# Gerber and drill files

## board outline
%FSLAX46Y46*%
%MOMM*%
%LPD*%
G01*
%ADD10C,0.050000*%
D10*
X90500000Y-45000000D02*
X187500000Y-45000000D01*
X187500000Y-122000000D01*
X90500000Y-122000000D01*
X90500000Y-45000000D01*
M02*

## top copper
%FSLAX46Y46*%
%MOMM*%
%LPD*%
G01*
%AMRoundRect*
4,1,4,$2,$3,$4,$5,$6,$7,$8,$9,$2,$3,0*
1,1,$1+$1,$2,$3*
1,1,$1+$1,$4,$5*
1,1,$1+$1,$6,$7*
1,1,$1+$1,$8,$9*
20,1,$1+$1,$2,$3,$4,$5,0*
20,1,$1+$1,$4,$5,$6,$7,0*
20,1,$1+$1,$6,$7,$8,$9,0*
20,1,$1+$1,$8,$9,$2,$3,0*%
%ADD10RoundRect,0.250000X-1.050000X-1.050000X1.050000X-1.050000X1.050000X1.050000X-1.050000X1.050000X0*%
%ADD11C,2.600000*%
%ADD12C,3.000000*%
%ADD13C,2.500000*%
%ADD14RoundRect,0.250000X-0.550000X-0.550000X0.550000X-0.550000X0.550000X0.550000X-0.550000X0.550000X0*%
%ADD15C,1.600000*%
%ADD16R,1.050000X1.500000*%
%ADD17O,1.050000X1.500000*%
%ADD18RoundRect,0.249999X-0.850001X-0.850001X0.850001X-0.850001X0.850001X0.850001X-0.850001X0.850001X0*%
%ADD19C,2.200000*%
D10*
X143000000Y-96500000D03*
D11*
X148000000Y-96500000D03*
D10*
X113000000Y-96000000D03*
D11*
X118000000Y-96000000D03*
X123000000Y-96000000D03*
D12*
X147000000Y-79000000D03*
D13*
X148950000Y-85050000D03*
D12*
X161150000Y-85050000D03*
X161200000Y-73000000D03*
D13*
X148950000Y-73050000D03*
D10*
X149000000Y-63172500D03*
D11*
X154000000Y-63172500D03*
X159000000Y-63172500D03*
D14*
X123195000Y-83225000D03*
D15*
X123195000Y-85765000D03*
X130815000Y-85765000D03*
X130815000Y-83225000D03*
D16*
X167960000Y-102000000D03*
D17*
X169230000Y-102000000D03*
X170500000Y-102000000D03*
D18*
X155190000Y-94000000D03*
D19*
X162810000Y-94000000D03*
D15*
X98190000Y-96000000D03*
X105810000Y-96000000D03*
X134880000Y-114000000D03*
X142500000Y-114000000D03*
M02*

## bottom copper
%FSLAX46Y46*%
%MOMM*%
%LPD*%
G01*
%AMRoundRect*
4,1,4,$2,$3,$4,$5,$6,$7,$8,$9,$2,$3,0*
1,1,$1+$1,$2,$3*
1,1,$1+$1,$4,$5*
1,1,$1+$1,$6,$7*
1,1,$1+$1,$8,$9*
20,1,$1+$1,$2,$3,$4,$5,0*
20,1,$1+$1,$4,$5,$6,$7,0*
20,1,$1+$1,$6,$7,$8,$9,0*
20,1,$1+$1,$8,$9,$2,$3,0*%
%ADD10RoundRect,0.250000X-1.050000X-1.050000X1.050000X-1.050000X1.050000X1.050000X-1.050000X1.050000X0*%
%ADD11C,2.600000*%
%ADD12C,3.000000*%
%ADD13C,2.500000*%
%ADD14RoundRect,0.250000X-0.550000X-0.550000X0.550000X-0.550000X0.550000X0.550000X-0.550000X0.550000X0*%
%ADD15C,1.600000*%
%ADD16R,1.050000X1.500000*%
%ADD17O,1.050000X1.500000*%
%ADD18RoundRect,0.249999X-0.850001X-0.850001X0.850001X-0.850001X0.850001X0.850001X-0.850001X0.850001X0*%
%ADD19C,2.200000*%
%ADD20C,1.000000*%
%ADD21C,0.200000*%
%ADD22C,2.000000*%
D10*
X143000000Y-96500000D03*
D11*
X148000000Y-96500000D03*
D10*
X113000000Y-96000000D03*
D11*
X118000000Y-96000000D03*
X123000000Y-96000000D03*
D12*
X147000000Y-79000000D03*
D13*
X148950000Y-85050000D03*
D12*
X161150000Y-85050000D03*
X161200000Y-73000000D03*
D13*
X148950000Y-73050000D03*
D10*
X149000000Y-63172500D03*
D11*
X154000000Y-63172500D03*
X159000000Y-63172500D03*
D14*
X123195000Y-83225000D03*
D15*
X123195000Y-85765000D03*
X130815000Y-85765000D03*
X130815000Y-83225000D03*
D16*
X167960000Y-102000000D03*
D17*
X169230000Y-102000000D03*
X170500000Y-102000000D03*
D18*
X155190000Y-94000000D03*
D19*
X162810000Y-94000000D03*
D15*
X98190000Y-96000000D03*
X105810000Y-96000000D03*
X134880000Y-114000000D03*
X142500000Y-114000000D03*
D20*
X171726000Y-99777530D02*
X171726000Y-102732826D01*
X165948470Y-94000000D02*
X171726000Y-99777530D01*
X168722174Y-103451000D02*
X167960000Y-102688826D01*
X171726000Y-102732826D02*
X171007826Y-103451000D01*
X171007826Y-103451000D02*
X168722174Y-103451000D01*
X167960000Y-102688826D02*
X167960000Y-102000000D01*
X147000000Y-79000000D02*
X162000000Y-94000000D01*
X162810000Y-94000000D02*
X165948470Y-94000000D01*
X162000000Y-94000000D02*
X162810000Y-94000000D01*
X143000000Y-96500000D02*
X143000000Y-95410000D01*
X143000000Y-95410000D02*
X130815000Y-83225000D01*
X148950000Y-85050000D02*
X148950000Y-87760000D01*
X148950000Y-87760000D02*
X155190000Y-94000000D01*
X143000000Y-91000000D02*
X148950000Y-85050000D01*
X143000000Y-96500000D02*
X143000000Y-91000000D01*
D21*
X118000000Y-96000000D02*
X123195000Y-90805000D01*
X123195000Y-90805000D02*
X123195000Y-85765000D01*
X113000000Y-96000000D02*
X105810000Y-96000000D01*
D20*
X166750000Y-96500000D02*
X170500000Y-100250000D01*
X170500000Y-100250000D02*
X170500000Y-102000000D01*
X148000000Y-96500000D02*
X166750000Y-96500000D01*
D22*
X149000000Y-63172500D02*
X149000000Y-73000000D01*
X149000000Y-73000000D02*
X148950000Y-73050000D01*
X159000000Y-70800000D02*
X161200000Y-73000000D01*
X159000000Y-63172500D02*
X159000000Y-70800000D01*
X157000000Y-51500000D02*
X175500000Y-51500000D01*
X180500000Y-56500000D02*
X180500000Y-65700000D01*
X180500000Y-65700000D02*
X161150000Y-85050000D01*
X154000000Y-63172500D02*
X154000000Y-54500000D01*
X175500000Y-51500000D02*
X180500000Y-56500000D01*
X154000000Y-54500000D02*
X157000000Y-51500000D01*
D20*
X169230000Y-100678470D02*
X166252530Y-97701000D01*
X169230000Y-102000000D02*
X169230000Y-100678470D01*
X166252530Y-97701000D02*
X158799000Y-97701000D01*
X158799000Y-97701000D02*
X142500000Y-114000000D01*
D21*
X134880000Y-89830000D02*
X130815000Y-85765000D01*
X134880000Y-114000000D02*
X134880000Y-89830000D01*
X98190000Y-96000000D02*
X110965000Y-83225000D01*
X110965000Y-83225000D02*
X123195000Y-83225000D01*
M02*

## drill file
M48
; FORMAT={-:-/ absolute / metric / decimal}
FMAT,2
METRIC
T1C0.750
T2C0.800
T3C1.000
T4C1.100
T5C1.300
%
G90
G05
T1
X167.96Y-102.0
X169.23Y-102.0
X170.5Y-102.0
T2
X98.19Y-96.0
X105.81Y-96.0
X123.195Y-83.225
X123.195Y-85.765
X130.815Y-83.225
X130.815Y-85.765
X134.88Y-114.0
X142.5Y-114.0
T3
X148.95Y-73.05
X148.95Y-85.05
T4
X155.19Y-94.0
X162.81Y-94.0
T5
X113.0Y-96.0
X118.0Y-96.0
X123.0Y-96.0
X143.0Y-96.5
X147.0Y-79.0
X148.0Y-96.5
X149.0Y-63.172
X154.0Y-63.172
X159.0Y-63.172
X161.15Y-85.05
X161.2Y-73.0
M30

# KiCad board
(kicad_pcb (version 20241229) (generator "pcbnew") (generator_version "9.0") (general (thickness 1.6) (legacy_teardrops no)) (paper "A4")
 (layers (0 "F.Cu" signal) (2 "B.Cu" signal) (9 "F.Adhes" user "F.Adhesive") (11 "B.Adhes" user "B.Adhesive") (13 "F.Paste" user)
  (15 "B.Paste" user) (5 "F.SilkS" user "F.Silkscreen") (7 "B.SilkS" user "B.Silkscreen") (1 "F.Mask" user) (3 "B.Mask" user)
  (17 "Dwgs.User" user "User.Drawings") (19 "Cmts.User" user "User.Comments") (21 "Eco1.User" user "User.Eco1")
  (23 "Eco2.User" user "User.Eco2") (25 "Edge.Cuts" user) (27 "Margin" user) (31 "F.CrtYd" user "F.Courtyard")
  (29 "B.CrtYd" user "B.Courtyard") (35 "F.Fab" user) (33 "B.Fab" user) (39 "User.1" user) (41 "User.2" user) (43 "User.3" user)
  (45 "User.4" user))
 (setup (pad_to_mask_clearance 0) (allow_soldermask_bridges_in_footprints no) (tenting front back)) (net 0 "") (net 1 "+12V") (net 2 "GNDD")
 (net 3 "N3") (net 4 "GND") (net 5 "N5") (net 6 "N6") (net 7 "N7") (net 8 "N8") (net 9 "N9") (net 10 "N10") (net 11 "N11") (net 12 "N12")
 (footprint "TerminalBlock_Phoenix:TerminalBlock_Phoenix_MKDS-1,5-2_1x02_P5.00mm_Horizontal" (layer "F.Cu") (at 143 96.5)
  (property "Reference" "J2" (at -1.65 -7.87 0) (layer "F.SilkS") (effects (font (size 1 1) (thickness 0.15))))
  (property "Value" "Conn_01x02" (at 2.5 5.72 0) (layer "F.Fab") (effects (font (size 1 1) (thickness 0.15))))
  (pad "1" thru_hole roundrect (at 0 0) (size 2.6 2.6) (drill 1.3) (layers "*.Cu" "*.Mask") (remove_unused_layers no)
   (roundrect_rratio 0.096154) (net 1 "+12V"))
  (pad "2" thru_hole circle (at 5 0) (size 2.6 2.6) (drill 1.3) (layers "*.Cu" "*.Mask") (remove_unused_layers no) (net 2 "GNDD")))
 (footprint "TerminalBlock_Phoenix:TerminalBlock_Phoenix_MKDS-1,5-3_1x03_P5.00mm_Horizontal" (layer "F.Cu") (at 113 96)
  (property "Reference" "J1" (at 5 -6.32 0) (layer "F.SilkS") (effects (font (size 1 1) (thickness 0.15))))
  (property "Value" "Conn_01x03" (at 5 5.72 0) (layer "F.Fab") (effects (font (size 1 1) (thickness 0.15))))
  (pad "1" thru_hole roundrect (at 0 0) (size 2.6 2.6) (drill 1.3) (layers "*.Cu" "*.Mask") (remove_unused_layers no)
   (roundrect_rratio 0.096154) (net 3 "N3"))
  (pad "2" thru_hole circle (at 5 0) (size 2.6 2.6) (drill 1.3) (layers "*.Cu" "*.Mask") (remove_unused_layers no) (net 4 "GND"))
  (pad "3" thru_hole circle (at 10 0) (size 2.6 2.6) (drill 1.3) (layers "*.Cu" "*.Mask") (remove_unused_layers no) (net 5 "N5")))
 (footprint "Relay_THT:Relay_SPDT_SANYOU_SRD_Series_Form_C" (layer "F.Cu") (at 147 79)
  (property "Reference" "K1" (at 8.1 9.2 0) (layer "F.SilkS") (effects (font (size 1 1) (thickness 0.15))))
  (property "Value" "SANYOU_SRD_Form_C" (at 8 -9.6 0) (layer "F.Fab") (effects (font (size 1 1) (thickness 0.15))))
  (pad "1" thru_hole circle (at 0 0 90) (size 3 3) (drill 1.3) (layers "*.Cu" "*.Mask") (remove_unused_layers no) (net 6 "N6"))
  (pad "2" thru_hole circle (at 1.95 6.05 90) (size 2.5 2.5) (drill 1) (layers "*.Cu" "*.Mask") (remove_unused_layers no) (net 1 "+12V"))
  (pad "3" thru_hole circle (at 14.15 6.05 90) (size 3 3) (drill 1.3) (layers "*.Cu" "*.Mask") (remove_unused_layers no) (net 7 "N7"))
  (pad "4" thru_hole circle (at 14.2 -6 90) (size 3 3) (drill 1.3) (layers "*.Cu" "*.Mask") (remove_unused_layers no) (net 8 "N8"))
  (pad "5" thru_hole circle (at 1.95 -5.95 90) (size 2.5 2.5) (drill 1) (layers "*.Cu" "*.Mask") (remove_unused_layers no) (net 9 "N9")))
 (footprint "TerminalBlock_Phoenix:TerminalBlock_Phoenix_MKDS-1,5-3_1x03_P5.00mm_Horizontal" (layer "F.Cu") (at 149 63.1725)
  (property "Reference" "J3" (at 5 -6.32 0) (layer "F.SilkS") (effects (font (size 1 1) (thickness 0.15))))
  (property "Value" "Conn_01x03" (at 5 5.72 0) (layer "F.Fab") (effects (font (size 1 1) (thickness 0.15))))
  (pad "1" thru_hole roundrect (at 0 0) (size 2.6 2.6) (drill 1.3) (layers "*.Cu" "*.Mask") (remove_unused_layers no)
   (roundrect_rratio 0.096154) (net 9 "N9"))
  (pad "2" thru_hole circle (at 5 0) (size 2.6 2.6) (drill 1.3) (layers "*.Cu" "*.Mask") (remove_unused_layers no) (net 7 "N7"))
  (pad "3" thru_hole circle (at 10 0) (size 2.6 2.6) (drill 1.3) (layers "*.Cu" "*.Mask") (remove_unused_layers no) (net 8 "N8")))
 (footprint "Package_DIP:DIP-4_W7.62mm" (layer "F.Cu") (at 123.195 83.225)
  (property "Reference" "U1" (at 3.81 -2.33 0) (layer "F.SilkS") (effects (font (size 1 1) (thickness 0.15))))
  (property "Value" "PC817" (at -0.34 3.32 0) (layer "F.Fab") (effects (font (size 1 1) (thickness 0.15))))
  (pad "1" thru_hole roundrect (at 0 0) (size 1.6 1.6) (drill 0.8) (layers "*.Cu" "*.Mask") (remove_unused_layers no)
   (roundrect_rratio 0.15625) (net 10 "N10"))
  (pad "2" thru_hole circle (at 0 2.54) (size 1.6 1.6) (drill 0.8) (layers "*.Cu" "*.Mask") (remove_unused_layers no) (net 4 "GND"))
  (pad "3" thru_hole circle (at 7.62 2.54) (size 1.6 1.6) (drill 0.8) (layers "*.Cu" "*.Mask") (remove_unused_layers no) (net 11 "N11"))
  (pad "4" thru_hole circle (at 7.62 0) (size 1.6 1.6) (drill 0.8) (layers "*.Cu" "*.Mask") (remove_unused_layers no) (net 1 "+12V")))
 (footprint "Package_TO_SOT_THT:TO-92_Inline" (layer "F.Cu") (at 167.96 102)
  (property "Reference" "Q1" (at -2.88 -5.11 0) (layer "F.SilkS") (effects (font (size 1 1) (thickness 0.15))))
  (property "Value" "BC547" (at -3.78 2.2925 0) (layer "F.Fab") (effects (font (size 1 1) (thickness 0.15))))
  (pad "1" thru_hole rect (at 0 0) (size 1.05 1.5) (drill 0.75) (layers "*.Cu" "*.Mask") (remove_unused_layers no) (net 6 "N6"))
  (pad "2" thru_hole oval (at 1.27 0) (size 1.05 1.5) (drill 0.75) (layers "*.Cu" "*.Mask") (remove_unused_layers no) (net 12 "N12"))
  (pad "3" thru_hole oval (at 2.54 0) (size 1.05 1.5) (drill 0.75) (layers "*.Cu" "*.Mask") (remove_unused_layers no) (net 2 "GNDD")))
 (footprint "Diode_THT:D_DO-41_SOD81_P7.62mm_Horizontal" (layer "F.Cu") (at 155.19 94)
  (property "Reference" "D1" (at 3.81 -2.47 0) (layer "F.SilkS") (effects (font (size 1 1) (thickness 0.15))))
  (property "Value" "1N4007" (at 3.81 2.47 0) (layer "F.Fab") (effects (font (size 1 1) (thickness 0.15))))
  (pad "1" thru_hole roundrect (at 0 0) (size 2.2 2.2) (drill 1.1) (layers "*.Cu" "*.Mask") (remove_unused_layers no)
   (roundrect_rratio 0.113636) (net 1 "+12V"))
  (pad "2" thru_hole circle (at 7.62 0) (size 2.2 2.2) (drill 1.1) (layers "*.Cu" "*.Mask") (remove_unused_layers no) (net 6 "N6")))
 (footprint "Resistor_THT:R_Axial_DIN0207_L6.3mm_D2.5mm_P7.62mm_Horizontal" (layer "F.Cu") (at 98.19 96)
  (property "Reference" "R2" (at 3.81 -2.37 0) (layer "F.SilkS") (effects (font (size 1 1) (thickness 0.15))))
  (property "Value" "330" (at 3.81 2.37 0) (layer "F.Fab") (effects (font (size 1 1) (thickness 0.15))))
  (pad "1" thru_hole circle (at 0 0) (size 1.6 1.6) (drill 0.8) (layers "*.Cu" "*.Mask") (remove_unused_layers no) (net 10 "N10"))
  (pad "2" thru_hole circle (at 7.62 0) (size 1.6 1.6) (drill 0.8) (layers "*.Cu" "*.Mask") (remove_unused_layers no) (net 3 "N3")))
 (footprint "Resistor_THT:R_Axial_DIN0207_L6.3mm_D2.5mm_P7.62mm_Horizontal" (layer "F.Cu") (at 134.88 114)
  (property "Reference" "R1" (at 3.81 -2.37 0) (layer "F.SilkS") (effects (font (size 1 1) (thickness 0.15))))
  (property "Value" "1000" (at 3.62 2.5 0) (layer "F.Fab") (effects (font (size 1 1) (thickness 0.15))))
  (pad "1" thru_hole circle (at 0 0) (size 1.6 1.6) (drill 0.8) (layers "*.Cu" "*.Mask") (remove_unused_layers no) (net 11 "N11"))
  (pad "2" thru_hole circle (at 7.62 0) (size 1.6 1.6) (drill 0.8) (layers "*.Cu" "*.Mask") (remove_unused_layers no) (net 12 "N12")))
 (gr_rect (start 90.5 45) (end 187.5 122) (stroke (width 0.05) (type default)) (fill no) (layer "Edge.Cuts"))
 (segment (start 171.726 99.77753) (end 171.726 102.732826) (width 1) (layer "B.Cu") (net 6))
 (segment (start 165.94847 94) (end 171.726 99.77753) (width 1) (layer "B.Cu") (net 6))
 (segment (start 168.722174 103.451) (end 167.96 102.688826) (width 1) (layer "B.Cu") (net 6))
 (segment (start 171.726 102.732826) (end 171.007826 103.451) (width 1) (layer "B.Cu") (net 6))
 (segment (start 171.007826 103.451) (end 168.722174 103.451) (width 1) (layer "B.Cu") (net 6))
 (segment (start 167.96 102.688826) (end 167.96 102) (width 1) (layer "B.Cu") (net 6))
 (segment (start 147 79) (end 162 94) (width 1) (layer "B.Cu") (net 6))
 (segment (start 162.81 94) (end 165.94847 94) (width 1) (layer "B.Cu") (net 6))
 (segment (start 162 94) (end 162.81 94) (width 1) (layer "B.Cu") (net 6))
 (segment (start 143 96.5) (end 143 95.41) (width 1) (layer "B.Cu") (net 1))
 (segment (start 143 95.41) (end 130.815 83.225) (width 1) (layer "B.Cu") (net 1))
 (segment (start 148.95 85.05) (end 148.95 87.76) (width 1) (layer "B.Cu") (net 1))
 (segment (start 148.95 87.76) (end 155.19 94) (width 1) (layer "B.Cu") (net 1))
 (segment (start 143 91) (end 148.95 85.05) (width 1) (layer "B.Cu") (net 1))
 (segment (start 143 96.5) (end 143 91) (width 1) (layer "B.Cu") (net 1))
 (segment (start 118 96) (end 123.195 90.805) (width 0.2) (layer "B.Cu") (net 4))
 (segment (start 123.195 90.805) (end 123.195 85.765) (width 0.2) (layer "B.Cu") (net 4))
 (segment (start 113 96) (end 105.81 96) (width 0.2) (layer "B.Cu") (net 3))
 (segment (start 166.75 96.5) (end 170.5 100.25) (width 1) (layer "B.Cu") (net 2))
 (segment (start 170.5 100.25) (end 170.5 102) (width 1) (layer "B.Cu") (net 2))
 (segment (start 148 96.5) (end 166.75 96.5) (width 1) (layer "B.Cu") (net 2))
 (segment (start 149 63.1725) (end 149 73) (width 2) (layer "B.Cu") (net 9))
 (segment (start 149 73) (end 148.95 73.05) (width 2) (layer "B.Cu") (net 9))
 (segment (start 159 70.8) (end 161.2 73) (width 2) (layer "B.Cu") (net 8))
 (segment (start 159 63.1725) (end 159 70.8) (width 2) (layer "B.Cu") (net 8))
 (segment (start 157 51.5) (end 175.5 51.5) (width 2) (layer "B.Cu") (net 7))
 (segment (start 180.5 56.5) (end 180.5 65.7) (width 2) (layer "B.Cu") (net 7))
 (segment (start 180.5 65.7) (end 161.15 85.05) (width 2) (layer "B.Cu") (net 7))
 (segment (start 154 63.1725) (end 154 54.5) (width 2) (layer "B.Cu") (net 7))
 (segment (start 175.5 51.5) (end 180.5 56.5) (width 2) (layer "B.Cu") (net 7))
 (segment (start 154 54.5) (end 157 51.5) (width 2) (layer "B.Cu") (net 7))
 (segment (start 169.23 100.67847) (end 166.25253 97.701) (width 1) (layer "B.Cu") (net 12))
 (segment (start 169.23 102) (end 169.23 100.67847) (width 1) (layer "B.Cu") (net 12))
 (segment (start 166.25253 97.701) (end 158.799 97.701) (width 1) (layer "B.Cu") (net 12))
 (segment (start 158.799 97.701) (end 142.5 114) (width 1) (layer "B.Cu") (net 12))
 (segment (start 134.88 89.83) (end 130.815 85.765) (width 0.2) (layer "B.Cu") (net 11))
 (segment (start 134.88 114) (end 134.88 89.83) (width 0.2) (layer "B.Cu") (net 11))
 (segment (start 98.19 96) (end 110.965 83.225) (width 0.2) (layer "B.Cu") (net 10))
 (segment (start 110.965 83.225) (end 123.195 83.225) (width 0.2) (layer "B.Cu") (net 10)))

